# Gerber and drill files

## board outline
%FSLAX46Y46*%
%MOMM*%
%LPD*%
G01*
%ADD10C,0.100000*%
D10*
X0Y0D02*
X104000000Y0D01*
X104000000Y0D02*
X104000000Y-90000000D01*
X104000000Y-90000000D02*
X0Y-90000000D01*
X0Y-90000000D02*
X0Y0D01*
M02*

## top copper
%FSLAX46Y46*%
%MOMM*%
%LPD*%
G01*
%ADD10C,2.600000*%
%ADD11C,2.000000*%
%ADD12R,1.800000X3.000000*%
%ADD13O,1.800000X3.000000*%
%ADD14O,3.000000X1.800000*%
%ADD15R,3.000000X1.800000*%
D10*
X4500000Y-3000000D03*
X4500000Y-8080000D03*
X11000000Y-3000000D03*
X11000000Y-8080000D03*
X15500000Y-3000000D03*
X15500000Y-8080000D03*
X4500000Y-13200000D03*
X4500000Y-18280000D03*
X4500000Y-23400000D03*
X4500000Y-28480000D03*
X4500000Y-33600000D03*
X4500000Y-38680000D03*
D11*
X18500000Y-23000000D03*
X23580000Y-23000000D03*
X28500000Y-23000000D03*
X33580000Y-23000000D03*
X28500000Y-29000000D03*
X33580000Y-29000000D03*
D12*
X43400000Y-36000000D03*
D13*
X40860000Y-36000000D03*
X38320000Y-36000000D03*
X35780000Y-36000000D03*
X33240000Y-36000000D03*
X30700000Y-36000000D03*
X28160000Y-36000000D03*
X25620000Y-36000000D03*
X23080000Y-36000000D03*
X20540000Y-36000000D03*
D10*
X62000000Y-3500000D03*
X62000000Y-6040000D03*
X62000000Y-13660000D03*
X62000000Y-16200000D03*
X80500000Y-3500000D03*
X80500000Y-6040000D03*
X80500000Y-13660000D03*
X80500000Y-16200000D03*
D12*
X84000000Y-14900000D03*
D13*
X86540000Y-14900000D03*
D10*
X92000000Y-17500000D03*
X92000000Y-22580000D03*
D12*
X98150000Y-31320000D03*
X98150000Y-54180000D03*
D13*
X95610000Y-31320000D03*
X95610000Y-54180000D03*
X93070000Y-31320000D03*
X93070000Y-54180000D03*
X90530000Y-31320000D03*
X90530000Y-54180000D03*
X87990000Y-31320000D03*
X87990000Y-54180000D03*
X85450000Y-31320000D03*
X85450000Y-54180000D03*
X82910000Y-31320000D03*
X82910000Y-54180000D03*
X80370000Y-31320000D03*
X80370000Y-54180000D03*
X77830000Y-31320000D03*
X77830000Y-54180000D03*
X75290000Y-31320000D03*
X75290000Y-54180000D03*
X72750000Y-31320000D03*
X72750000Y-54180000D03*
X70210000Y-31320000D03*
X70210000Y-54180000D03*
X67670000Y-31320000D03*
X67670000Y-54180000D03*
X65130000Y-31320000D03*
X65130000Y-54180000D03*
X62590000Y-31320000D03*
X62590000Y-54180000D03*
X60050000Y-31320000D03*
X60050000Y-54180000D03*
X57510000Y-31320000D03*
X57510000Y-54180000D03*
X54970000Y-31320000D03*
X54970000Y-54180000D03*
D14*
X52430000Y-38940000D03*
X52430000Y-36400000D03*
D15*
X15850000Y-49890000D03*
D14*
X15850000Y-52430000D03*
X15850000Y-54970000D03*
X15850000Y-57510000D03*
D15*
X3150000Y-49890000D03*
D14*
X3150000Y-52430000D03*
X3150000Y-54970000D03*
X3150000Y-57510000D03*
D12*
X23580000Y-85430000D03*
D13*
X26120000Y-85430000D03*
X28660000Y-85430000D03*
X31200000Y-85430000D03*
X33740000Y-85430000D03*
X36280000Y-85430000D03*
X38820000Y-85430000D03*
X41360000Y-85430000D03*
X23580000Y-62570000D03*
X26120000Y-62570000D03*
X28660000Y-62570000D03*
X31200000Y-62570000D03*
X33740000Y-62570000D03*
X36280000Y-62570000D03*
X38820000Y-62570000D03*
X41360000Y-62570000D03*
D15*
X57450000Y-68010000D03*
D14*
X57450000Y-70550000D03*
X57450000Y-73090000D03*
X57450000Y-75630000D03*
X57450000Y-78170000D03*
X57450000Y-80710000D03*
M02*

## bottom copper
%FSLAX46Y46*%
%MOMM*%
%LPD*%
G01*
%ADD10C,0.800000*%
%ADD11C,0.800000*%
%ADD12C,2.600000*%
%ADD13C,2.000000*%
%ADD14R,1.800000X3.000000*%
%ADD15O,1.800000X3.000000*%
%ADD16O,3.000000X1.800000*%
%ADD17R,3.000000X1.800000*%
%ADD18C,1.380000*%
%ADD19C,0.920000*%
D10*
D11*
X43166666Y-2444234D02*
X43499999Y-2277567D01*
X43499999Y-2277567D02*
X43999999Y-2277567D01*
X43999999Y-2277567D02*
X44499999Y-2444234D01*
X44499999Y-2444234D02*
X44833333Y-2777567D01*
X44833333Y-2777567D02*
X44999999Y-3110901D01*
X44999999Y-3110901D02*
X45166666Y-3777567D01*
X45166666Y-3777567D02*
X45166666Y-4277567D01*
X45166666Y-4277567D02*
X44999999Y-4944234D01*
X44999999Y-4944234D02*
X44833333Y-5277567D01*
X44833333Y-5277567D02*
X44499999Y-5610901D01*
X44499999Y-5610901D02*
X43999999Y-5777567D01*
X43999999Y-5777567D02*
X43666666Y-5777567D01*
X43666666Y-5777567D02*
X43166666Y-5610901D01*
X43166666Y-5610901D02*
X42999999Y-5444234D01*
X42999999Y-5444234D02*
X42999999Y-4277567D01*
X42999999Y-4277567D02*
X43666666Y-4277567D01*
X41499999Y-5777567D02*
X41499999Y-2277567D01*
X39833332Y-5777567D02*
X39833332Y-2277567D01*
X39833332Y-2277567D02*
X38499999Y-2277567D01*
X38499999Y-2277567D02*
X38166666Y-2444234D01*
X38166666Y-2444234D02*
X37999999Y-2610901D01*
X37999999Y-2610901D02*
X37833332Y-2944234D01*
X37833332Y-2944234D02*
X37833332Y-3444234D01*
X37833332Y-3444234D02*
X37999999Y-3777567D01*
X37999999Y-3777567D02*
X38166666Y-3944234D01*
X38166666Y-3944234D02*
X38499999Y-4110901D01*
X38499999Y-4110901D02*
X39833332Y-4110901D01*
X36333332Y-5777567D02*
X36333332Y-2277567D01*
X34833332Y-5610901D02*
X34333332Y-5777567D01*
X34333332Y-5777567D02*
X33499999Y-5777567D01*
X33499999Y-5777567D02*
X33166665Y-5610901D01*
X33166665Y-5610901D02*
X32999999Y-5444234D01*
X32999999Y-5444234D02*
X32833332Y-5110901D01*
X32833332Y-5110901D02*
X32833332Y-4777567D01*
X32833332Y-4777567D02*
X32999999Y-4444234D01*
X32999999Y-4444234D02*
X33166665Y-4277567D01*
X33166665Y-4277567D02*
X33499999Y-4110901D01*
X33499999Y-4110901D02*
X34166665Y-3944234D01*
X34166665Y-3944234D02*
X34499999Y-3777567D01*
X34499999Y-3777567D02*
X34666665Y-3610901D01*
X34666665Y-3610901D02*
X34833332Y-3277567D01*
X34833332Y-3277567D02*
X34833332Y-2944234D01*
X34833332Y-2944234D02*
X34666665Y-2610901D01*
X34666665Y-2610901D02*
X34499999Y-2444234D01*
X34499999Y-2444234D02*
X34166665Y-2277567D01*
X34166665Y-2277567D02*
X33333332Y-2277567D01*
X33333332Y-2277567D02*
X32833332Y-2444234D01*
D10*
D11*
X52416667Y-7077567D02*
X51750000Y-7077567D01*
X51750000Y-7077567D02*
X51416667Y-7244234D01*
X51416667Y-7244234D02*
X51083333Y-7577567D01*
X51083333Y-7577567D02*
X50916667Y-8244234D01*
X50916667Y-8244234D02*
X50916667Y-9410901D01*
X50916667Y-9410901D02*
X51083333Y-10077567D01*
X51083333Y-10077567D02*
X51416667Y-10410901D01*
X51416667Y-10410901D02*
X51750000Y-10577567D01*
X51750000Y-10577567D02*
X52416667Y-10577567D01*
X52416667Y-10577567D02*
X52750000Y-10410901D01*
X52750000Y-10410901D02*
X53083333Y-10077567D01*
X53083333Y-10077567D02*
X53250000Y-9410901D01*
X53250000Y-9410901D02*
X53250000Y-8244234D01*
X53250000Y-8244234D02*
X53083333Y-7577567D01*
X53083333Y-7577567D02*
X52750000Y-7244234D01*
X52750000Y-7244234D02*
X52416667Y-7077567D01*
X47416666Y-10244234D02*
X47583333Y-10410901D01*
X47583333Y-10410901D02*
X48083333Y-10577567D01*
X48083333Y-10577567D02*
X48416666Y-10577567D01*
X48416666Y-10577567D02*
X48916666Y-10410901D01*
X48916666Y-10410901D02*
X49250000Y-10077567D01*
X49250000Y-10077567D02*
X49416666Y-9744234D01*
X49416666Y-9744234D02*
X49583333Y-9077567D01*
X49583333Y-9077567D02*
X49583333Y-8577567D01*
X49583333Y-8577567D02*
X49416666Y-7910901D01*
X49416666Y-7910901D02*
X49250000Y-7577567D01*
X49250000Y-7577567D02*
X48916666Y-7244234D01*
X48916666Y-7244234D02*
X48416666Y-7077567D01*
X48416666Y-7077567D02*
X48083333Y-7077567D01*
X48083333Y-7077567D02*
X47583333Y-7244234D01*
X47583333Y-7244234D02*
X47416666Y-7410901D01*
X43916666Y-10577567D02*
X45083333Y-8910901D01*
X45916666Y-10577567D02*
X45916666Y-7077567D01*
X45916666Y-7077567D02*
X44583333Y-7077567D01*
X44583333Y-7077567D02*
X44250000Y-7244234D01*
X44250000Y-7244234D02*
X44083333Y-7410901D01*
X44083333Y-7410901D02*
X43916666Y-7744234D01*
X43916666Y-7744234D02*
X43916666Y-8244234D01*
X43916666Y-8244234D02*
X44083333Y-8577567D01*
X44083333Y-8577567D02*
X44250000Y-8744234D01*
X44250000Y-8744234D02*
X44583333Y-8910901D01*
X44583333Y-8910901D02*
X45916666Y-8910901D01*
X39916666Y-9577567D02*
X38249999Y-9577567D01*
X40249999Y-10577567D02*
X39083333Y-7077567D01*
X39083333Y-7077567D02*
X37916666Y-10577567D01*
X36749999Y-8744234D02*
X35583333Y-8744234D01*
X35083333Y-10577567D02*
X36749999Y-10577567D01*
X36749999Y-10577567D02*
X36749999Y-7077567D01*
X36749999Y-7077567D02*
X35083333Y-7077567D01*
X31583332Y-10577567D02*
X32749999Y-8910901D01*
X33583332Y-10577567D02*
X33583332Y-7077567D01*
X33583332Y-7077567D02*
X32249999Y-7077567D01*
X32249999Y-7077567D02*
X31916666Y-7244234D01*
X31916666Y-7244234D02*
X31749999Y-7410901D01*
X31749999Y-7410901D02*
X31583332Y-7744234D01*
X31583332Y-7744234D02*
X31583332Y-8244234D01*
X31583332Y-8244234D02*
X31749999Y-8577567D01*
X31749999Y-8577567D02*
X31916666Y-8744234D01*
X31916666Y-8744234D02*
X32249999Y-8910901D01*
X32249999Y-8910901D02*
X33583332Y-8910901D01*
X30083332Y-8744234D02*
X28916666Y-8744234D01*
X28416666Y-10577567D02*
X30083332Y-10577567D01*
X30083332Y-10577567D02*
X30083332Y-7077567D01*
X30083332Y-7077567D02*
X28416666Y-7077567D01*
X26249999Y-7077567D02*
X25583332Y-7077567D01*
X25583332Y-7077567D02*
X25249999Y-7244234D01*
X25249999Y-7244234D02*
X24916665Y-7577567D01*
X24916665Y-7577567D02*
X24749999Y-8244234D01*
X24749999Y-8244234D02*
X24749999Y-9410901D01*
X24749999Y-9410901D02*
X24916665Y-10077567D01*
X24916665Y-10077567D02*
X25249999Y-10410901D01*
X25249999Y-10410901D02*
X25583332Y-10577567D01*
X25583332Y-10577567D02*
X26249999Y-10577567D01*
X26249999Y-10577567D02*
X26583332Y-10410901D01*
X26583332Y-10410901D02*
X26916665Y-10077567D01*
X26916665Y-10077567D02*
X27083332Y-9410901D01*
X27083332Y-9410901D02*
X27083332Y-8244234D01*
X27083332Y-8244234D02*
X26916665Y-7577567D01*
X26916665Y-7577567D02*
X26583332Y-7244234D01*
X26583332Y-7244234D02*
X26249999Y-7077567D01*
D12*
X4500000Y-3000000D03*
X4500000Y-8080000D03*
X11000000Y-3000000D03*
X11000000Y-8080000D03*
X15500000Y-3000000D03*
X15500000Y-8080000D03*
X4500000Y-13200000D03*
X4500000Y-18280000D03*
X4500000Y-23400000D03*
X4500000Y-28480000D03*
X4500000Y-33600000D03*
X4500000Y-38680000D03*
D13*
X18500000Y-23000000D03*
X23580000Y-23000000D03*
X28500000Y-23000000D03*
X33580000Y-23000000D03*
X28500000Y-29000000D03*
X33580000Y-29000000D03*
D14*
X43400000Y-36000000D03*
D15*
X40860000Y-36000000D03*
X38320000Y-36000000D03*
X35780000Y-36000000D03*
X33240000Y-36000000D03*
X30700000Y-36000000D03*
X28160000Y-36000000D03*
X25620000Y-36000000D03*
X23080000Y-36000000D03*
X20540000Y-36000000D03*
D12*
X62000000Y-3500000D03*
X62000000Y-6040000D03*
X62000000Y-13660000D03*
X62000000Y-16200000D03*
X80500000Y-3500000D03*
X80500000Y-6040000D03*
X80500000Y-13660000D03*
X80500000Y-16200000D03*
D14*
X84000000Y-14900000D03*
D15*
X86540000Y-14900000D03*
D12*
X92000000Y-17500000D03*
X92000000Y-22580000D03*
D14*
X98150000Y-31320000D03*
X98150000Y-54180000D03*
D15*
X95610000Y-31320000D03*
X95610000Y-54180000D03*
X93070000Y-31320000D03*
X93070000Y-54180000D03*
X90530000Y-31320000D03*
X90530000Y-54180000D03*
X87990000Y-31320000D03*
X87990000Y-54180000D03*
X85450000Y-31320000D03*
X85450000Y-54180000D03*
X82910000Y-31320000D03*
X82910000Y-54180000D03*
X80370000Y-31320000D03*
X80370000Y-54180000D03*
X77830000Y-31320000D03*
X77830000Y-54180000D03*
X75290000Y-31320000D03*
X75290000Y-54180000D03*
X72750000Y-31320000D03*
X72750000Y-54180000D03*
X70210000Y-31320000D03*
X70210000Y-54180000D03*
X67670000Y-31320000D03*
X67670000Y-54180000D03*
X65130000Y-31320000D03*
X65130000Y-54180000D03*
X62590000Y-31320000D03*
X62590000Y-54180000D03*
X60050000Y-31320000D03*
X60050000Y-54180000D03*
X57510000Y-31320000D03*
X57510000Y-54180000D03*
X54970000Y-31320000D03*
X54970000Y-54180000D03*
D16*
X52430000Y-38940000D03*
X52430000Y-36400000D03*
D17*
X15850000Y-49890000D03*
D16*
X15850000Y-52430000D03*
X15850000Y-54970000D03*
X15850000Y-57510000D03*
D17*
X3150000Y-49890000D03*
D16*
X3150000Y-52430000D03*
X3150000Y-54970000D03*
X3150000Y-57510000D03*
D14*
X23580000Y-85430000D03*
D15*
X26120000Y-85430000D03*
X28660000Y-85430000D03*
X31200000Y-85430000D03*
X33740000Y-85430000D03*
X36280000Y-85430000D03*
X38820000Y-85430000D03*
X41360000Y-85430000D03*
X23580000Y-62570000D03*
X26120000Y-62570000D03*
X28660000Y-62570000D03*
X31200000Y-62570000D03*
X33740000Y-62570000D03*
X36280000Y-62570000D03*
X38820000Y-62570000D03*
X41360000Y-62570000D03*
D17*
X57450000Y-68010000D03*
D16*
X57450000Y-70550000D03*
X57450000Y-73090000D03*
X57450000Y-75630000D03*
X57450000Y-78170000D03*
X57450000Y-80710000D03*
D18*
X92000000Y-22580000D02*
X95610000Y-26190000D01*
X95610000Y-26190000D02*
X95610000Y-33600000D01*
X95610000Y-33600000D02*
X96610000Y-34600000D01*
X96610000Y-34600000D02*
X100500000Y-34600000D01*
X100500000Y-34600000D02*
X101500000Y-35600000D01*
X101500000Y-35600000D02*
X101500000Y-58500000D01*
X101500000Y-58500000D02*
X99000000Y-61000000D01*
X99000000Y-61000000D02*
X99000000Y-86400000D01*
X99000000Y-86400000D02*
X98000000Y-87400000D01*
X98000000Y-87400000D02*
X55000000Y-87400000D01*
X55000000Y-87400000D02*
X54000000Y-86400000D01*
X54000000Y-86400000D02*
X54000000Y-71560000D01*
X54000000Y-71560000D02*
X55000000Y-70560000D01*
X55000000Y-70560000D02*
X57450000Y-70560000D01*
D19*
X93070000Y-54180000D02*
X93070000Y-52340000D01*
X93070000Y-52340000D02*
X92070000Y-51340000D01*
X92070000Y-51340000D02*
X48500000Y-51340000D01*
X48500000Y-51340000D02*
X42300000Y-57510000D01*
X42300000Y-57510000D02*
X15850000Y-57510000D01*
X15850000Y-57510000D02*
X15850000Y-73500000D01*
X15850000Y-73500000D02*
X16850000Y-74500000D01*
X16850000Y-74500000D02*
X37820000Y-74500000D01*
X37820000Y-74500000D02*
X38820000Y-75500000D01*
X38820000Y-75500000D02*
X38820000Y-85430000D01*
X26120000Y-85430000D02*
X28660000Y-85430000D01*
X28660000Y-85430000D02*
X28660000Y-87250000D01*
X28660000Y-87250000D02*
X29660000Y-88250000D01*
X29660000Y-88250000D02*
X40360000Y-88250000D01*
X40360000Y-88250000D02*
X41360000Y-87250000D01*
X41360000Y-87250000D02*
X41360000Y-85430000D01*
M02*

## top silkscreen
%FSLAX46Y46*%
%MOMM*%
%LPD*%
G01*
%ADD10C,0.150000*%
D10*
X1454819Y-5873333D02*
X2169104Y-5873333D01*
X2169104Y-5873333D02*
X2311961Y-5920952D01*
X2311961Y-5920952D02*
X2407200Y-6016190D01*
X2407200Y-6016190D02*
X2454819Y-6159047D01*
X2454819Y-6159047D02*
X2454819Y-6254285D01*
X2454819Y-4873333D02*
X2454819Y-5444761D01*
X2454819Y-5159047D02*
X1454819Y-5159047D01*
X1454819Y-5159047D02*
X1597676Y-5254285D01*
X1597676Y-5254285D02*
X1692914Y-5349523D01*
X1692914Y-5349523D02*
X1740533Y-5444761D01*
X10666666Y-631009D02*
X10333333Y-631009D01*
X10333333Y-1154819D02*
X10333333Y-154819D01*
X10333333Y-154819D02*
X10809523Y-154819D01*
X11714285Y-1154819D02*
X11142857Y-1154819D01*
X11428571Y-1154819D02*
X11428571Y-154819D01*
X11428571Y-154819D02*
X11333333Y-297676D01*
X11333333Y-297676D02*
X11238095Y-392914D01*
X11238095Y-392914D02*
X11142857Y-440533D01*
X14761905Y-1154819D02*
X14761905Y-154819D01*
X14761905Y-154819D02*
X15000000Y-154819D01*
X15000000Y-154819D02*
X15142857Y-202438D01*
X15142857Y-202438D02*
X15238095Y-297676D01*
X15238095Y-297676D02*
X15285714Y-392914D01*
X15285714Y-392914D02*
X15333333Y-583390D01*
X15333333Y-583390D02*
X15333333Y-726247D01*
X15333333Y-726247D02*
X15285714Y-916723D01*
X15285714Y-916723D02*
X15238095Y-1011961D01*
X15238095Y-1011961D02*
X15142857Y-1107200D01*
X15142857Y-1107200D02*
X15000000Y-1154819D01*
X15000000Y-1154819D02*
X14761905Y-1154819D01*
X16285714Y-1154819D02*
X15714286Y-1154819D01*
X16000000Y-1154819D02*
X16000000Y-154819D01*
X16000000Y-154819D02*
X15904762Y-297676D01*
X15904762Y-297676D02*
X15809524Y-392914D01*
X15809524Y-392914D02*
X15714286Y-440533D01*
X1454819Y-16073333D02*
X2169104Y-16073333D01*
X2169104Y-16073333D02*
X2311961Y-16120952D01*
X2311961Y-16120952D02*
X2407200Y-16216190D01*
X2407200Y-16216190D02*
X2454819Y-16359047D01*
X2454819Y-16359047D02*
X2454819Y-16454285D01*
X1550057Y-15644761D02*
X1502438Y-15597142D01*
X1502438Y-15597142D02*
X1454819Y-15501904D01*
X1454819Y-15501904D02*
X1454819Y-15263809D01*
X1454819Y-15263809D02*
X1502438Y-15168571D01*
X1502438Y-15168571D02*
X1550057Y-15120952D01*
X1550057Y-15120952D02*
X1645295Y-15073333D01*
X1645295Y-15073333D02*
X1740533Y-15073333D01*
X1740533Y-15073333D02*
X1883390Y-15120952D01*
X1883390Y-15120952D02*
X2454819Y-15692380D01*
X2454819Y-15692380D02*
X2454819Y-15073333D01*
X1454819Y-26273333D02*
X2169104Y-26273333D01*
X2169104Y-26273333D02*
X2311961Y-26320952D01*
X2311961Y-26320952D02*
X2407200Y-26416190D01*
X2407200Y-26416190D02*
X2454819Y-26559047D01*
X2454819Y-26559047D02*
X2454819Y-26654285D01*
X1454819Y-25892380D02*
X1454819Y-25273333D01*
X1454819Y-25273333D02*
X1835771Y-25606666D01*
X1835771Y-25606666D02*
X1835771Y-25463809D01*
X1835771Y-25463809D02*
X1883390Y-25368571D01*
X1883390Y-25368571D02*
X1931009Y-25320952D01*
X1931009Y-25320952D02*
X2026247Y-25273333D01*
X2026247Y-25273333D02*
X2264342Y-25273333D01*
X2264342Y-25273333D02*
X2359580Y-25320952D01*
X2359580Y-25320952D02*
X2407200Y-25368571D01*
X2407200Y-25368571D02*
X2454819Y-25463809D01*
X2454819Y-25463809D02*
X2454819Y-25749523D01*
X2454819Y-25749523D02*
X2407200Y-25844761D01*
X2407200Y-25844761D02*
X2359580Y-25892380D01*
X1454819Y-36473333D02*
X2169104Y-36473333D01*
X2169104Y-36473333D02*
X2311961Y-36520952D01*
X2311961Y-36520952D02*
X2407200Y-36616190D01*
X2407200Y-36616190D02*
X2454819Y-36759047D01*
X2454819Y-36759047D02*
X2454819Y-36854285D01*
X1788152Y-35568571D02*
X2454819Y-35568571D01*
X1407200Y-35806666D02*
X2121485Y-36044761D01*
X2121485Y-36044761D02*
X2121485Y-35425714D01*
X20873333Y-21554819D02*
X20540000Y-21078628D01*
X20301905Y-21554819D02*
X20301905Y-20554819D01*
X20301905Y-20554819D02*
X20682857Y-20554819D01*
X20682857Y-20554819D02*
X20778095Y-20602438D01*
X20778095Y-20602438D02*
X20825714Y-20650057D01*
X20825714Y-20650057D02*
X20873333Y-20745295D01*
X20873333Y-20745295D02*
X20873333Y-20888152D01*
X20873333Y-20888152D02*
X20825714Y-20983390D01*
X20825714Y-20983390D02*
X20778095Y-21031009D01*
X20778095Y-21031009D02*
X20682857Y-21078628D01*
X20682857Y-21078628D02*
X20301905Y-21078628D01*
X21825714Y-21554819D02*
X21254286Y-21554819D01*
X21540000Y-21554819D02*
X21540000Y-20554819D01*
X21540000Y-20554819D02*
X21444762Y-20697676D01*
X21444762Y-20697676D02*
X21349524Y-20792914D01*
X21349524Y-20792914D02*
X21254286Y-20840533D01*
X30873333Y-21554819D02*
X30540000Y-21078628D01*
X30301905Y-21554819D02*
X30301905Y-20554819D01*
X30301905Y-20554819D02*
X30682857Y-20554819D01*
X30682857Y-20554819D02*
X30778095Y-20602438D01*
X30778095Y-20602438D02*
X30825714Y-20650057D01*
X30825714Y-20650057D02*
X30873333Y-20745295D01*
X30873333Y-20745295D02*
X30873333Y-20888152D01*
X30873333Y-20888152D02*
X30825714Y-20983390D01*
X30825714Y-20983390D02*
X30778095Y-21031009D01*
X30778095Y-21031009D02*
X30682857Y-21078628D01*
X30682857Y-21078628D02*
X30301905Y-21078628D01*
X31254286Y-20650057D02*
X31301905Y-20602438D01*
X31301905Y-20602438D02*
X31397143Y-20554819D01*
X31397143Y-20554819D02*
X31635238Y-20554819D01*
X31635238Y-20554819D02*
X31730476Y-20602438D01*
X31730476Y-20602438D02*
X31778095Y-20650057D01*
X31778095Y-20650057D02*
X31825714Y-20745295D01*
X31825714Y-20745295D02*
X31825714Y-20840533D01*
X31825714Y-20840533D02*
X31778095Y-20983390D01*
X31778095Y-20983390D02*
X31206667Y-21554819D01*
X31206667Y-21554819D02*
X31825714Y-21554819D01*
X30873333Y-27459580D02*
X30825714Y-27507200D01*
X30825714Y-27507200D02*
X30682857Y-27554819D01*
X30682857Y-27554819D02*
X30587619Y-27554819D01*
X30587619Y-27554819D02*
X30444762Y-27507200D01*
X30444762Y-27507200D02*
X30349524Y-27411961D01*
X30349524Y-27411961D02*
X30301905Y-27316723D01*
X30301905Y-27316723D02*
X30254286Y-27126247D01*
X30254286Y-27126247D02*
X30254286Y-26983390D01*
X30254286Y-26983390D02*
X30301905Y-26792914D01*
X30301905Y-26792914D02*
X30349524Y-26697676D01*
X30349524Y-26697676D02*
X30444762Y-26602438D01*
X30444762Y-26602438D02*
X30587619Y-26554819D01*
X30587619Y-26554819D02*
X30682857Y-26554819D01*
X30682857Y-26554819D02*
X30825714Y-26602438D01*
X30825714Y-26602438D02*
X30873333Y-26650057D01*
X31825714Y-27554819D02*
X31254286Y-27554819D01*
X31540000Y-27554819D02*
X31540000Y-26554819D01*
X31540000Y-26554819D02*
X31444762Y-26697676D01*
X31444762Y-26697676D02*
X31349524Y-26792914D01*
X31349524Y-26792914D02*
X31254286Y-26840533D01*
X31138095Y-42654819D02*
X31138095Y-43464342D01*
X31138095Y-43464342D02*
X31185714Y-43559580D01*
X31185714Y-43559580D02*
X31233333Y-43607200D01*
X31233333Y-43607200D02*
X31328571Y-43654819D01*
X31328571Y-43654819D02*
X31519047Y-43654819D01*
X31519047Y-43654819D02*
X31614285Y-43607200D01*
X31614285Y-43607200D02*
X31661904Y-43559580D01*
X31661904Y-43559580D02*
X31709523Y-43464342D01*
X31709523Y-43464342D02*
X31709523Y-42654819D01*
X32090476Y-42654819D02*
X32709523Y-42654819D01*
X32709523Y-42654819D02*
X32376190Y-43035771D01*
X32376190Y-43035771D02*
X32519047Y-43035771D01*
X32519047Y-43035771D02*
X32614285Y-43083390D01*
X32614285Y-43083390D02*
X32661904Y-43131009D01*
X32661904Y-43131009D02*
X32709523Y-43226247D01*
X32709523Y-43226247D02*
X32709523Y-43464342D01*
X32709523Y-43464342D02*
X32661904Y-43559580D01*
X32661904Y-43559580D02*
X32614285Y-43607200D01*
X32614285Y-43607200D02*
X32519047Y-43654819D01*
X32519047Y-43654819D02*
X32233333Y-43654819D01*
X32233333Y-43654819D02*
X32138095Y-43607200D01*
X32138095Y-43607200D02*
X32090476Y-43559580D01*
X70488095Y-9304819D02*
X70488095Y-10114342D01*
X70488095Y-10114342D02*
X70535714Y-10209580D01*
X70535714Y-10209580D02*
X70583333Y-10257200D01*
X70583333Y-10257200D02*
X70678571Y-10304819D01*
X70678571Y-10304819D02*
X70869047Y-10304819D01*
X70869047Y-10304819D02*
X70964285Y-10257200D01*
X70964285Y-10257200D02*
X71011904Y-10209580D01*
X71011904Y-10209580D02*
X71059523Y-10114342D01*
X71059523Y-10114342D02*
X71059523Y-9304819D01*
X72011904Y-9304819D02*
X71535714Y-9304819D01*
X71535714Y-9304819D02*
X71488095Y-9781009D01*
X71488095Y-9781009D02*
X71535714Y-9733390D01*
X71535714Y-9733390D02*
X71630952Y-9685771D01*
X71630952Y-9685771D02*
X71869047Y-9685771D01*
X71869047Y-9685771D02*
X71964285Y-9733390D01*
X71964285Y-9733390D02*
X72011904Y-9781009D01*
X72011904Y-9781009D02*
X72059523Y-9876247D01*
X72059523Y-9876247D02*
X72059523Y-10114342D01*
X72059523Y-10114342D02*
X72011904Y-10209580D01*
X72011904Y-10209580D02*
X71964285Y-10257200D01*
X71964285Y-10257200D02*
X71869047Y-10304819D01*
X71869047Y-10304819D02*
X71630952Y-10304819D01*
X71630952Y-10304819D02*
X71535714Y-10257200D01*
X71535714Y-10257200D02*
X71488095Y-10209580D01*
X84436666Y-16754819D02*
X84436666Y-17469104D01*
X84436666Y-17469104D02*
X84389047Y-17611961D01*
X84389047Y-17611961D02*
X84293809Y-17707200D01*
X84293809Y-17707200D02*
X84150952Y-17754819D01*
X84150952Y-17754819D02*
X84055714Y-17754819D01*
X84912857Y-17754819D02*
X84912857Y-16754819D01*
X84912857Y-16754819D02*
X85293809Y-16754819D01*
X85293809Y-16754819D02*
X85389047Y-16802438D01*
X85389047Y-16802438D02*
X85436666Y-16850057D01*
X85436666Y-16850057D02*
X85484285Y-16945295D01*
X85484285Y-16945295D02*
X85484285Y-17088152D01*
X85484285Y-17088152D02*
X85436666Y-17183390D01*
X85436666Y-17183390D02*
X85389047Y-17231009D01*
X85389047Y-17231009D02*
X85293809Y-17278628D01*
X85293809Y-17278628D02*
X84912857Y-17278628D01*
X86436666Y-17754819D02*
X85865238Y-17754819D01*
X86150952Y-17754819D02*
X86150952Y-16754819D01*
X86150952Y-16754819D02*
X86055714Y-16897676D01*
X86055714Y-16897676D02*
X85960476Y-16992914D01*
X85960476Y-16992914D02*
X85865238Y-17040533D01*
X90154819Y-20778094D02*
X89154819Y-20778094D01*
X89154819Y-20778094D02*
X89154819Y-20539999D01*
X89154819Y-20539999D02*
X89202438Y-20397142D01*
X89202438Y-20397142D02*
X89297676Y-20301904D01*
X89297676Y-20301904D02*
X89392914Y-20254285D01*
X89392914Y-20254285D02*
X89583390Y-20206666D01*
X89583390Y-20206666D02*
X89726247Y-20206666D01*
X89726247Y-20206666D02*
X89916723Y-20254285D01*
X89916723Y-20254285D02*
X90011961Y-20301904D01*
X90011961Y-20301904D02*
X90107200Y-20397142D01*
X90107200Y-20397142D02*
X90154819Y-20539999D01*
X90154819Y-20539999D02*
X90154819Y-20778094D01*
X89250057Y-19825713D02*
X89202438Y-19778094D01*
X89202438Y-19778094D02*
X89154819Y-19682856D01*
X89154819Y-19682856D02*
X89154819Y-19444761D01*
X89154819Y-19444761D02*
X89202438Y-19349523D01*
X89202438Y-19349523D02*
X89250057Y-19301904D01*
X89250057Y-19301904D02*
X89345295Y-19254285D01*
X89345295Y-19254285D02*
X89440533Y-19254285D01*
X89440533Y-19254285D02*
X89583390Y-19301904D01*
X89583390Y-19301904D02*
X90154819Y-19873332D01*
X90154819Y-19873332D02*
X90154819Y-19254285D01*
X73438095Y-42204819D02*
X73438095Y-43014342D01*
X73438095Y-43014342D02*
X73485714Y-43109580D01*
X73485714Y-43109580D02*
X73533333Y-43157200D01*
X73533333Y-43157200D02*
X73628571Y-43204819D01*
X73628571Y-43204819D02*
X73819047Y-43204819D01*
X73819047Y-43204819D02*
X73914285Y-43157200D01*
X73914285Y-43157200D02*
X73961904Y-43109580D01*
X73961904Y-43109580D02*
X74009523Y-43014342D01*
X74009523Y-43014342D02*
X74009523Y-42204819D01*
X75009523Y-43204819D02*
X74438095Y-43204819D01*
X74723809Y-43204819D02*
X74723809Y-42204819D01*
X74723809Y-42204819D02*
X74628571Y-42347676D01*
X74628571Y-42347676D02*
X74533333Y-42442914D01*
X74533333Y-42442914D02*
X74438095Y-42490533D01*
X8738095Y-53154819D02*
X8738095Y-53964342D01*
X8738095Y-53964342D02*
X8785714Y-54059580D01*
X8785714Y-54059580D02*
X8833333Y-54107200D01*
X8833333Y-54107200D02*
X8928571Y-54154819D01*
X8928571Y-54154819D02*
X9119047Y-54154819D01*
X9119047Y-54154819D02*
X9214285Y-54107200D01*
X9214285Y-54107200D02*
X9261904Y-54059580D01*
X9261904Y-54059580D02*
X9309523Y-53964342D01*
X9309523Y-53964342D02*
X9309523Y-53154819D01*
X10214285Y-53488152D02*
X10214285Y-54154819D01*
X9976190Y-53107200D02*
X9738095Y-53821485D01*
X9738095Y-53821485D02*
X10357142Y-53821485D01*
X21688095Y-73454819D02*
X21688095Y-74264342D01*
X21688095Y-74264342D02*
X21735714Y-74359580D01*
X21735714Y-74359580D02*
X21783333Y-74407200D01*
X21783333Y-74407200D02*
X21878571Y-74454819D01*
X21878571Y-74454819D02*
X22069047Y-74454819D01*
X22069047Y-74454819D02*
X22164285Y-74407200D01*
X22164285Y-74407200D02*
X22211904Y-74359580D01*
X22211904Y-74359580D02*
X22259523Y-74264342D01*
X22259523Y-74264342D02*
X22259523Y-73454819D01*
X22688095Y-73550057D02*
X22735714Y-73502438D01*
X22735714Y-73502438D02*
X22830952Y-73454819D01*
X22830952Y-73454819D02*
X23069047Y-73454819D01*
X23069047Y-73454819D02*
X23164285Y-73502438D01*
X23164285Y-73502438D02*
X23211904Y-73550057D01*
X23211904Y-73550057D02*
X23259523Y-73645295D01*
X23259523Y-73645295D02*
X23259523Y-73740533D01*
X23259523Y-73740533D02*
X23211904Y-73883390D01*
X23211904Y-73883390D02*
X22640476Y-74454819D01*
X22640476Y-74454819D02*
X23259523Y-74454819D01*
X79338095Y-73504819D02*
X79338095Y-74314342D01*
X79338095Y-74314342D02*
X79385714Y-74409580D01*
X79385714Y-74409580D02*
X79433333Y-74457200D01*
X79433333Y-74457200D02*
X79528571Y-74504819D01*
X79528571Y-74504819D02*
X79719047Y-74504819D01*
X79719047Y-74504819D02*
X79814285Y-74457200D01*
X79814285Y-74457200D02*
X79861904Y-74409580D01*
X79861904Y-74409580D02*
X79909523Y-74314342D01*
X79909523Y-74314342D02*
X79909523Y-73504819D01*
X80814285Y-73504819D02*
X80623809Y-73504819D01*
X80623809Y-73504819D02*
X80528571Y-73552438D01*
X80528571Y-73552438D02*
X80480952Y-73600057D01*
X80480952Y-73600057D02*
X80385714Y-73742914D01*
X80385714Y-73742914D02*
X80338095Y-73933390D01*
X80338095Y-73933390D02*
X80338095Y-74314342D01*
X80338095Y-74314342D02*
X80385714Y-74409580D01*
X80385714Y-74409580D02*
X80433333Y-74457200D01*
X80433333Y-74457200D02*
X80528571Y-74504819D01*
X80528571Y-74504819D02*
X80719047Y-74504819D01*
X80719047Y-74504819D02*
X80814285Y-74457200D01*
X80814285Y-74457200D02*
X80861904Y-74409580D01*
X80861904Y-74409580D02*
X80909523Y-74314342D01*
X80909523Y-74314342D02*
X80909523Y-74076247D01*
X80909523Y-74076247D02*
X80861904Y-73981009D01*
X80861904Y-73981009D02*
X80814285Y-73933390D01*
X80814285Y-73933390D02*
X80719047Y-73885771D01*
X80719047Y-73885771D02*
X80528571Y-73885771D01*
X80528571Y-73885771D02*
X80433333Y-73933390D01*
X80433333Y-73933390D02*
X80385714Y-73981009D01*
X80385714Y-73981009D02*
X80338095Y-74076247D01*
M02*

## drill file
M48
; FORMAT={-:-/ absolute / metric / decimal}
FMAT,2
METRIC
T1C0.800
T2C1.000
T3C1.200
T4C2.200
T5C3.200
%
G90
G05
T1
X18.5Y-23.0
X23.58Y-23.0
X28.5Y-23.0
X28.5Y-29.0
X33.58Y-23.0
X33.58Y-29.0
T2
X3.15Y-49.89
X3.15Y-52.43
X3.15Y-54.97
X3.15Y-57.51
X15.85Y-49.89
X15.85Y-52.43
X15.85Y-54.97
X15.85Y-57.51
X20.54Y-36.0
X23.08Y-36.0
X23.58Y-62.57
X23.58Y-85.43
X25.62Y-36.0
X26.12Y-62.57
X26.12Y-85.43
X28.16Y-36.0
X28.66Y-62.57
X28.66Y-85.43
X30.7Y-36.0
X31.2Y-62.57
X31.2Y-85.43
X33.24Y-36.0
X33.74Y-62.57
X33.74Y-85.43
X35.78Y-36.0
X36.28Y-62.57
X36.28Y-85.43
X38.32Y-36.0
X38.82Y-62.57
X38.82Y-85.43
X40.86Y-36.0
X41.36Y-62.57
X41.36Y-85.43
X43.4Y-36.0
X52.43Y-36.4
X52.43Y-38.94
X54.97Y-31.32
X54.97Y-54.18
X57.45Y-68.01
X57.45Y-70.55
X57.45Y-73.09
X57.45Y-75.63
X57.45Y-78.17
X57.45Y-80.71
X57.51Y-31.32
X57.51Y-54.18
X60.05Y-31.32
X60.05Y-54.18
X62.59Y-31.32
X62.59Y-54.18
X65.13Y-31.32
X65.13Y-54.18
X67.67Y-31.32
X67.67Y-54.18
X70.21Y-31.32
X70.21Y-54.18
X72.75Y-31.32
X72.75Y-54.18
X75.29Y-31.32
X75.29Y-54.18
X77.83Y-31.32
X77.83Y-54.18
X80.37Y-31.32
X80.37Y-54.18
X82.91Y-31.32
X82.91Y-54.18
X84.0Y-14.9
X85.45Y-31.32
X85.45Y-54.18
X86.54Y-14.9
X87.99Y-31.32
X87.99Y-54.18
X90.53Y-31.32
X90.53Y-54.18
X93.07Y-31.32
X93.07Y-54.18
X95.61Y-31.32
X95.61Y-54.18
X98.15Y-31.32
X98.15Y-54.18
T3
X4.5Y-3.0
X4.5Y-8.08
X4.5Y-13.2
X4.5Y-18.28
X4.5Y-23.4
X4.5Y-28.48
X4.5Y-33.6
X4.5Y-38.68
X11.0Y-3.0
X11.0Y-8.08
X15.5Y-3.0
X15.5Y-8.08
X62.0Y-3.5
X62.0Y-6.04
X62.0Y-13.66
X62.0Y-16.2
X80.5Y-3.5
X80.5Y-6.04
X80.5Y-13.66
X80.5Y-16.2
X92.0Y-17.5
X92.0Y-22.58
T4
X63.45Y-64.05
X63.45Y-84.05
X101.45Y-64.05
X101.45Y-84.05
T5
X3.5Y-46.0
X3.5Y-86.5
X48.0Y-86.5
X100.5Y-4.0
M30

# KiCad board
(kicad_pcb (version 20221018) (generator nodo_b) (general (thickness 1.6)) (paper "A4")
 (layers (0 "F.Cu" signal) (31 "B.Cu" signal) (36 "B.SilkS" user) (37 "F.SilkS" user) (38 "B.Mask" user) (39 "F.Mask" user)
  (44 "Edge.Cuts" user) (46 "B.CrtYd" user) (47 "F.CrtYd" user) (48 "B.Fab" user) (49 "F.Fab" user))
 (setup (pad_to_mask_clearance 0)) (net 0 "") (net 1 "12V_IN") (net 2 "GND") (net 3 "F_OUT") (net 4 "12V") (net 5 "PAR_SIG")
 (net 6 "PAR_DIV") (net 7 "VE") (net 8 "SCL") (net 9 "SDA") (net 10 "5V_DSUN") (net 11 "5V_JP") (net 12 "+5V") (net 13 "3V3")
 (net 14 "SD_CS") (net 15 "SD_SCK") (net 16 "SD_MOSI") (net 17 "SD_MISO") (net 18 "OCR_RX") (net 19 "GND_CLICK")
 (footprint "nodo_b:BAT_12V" (layer "F.Cu") (at 4.5 3.0)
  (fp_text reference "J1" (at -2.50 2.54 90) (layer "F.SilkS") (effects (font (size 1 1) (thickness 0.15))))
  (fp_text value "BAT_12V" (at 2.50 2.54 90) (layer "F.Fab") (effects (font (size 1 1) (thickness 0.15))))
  (pad "1" thru_hole circle (at 0 0.0) (size 2.6 2.6) (drill 1.2) (layers "*.Cu" "*.Mask") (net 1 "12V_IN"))
  (pad "2" thru_hole circle (at 0 5.08) (size 2.6 2.6) (drill 1.2) (layers "*.Cu" "*.Mask") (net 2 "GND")))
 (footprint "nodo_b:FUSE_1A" (layer "F.Cu") (at 11.0 3.0)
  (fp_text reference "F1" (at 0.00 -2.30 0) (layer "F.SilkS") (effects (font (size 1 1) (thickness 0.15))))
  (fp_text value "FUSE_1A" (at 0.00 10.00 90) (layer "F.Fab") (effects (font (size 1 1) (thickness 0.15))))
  (pad "1" thru_hole circle (at 0 0) (size 2.6 2.6) (drill 1.2) (layers "*.Cu" "*.Mask") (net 1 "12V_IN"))
  (pad "2" thru_hole circle (at 0 5.08) (size 2.6 2.6) (drill 1.2) (layers "*.Cu" "*.Mask") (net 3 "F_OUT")))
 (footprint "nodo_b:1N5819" (layer "F.Cu") (at 15.5 3.0)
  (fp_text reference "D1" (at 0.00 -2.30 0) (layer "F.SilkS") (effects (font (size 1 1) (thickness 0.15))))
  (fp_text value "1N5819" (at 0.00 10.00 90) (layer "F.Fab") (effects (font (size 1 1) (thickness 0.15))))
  (pad "1" thru_hole circle (at 0 0) (size 2.6 2.6) (drill 1.2) (layers "*.Cu" "*.Mask") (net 3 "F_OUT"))
  (pad "2" thru_hole circle (at 0 5.08) (size 2.6 2.6) (drill 1.2) (layers "*.Cu" "*.Mask") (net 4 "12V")))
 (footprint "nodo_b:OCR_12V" (layer "F.Cu") (at 4.5 13.2)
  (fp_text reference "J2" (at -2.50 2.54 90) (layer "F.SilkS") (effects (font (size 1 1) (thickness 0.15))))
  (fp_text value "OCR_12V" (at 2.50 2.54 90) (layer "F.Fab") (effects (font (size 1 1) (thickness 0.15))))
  (pad "1" thru_hole circle (at 0 0.0) (size 2.6 2.6) (drill 1.2) (layers "*.Cu" "*.Mask") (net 2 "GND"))
  (pad "2" thru_hole circle (at 0 5.08) (size 2.6 2.6) (drill 1.2) (layers "*.Cu" "*.Mask") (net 4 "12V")))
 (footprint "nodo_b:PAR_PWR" (layer "F.Cu") (at 4.5 23.4)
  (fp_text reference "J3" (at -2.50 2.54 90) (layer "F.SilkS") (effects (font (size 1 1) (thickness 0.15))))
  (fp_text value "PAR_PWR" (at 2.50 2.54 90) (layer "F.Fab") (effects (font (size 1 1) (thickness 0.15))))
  (pad "1" thru_hole circle (at 0 0.0) (size 2.6 2.6) (drill 1.2) (layers "*.Cu" "*.Mask") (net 4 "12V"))
  (pad "2" thru_hole circle (at 0 5.08) (size 2.6 2.6) (drill 1.2) (layers "*.Cu" "*.Mask") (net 2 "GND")))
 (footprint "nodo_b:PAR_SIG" (layer "F.Cu") (at 4.5 33.6)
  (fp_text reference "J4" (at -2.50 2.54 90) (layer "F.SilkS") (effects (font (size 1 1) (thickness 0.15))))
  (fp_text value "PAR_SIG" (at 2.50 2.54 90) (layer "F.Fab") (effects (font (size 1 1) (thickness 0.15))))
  (pad "1" thru_hole circle (at 0 0.0) (size 2.6 2.6) (drill 1.2) (layers "*.Cu" "*.Mask") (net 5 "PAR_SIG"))
  (pad "2" thru_hole circle (at 0 5.08) (size 2.6 2.6) (drill 1.2) (layers "*.Cu" "*.Mask") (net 2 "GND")))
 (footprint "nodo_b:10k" (layer "F.Cu") (at 18.5 23.0)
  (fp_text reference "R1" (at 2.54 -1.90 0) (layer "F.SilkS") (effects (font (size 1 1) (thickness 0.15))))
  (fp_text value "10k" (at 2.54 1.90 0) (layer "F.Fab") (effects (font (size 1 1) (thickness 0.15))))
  (pad "1" thru_hole circle (at 0 0) (size 2.0 2.0) (drill 0.8) (layers "*.Cu" "*.Mask") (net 5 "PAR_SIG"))
  (pad "2" thru_hole circle (at 5.08 0) (size 2.0 2.0) (drill 0.8) (layers "*.Cu" "*.Mask") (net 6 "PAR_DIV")))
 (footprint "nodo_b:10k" (layer "F.Cu") (at 28.5 23.0)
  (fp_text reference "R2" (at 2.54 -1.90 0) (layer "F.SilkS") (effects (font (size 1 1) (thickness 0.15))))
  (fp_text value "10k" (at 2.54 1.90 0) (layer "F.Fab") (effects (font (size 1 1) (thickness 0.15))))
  (pad "1" thru_hole circle (at 0 0) (size 2.0 2.0) (drill 0.8) (layers "*.Cu" "*.Mask") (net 2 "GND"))
  (pad "2" thru_hole circle (at 5.08 0) (size 2.0 2.0) (drill 0.8) (layers "*.Cu" "*.Mask") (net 6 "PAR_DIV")))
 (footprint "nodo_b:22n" (layer "F.Cu") (at 28.5 29.0)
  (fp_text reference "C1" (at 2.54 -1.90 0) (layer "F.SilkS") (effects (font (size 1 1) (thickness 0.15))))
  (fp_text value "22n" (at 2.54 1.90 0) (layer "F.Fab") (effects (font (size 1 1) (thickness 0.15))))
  (pad "1" thru_hole circle (at 0 0) (size 2.0 2.0) (drill 0.8) (layers "*.Cu" "*.Mask") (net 6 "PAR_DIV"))
  (pad "2" thru_hole circle (at 5.08 0) (size 2.0 2.0) (drill 0.8) (layers "*.Cu" "*.Mask") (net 2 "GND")))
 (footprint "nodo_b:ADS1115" (layer "F.Cu") (at 43.4 36.0 180)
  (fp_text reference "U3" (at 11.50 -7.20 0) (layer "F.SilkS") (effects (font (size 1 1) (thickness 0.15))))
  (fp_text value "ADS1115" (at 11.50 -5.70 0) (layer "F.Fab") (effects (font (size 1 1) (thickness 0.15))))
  (pad "1" thru_hole rect (at 0.0 0 180) (size 1.8 3.0) (drill 1.0) (layers "*.Cu" "*.Mask") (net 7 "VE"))
  (pad "2" thru_hole oval (at 2.54 0 180) (size 1.8 3.0) (drill 1.0) (layers "*.Cu" "*.Mask") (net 2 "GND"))
  (pad "3" thru_hole oval (at 5.08 0 180) (size 1.8 3.0) (drill 1.0) (layers "*.Cu" "*.Mask") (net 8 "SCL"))
  (pad "4" thru_hole oval (at 7.62 0 180) (size 1.8 3.0) (drill 1.0) (layers "*.Cu" "*.Mask") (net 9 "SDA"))
  (pad "5" thru_hole oval (at 10.16 0 180) (size 1.8 3.0) (drill 1.0) (layers "*.Cu" "*.Mask") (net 2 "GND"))
  (pad "6" thru_hole oval (at 12.7 0 180) (size 1.8 3.0) (drill 1.0) (layers "*.Cu" "*.Mask"))
  (pad "7" thru_hole oval (at 15.24 0 180) (size 1.8 3.0) (drill 1.0) (layers "*.Cu" "*.Mask") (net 6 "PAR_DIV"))
  (pad "8" thru_hole oval (at 17.78 0 180) (size 1.8 3.0) (drill 1.0) (layers "*.Cu" "*.Mask"))
  (pad "9" thru_hole oval (at 20.32 0 180) (size 1.8 3.0) (drill 1.0) (layers "*.Cu" "*.Mask"))
  (pad "10" thru_hole oval (at 22.86 0 180) (size 1.8 3.0) (drill 1.0) (layers "*.Cu" "*.Mask")))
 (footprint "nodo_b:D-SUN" (layer "F.Cu") (at 62.0 3.5)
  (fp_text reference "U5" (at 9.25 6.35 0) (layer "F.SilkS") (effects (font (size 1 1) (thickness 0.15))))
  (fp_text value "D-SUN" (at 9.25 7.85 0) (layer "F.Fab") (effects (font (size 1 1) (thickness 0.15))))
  (pad "1" thru_hole circle (at 0 0.0) (size 2.6 2.6) (drill 1.2) (layers "*.Cu" "*.Mask") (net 2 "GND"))
  (pad "2" thru_hole circle (at 0 2.54) (size 2.6 2.6) (drill 1.2) (layers "*.Cu" "*.Mask") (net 2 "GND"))
  (pad "3" thru_hole circle (at 0 10.16) (size 2.6 2.6) (drill 1.2) (layers "*.Cu" "*.Mask") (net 4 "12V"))
  (pad "4" thru_hole circle (at 0 12.7) (size 2.6 2.6) (drill 1.2) (layers "*.Cu" "*.Mask") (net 4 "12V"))
  (pad "5" thru_hole circle (at 18.5 0.0) (size 2.6 2.6) (drill 1.2) (layers "*.Cu" "*.Mask") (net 2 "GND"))
  (pad "6" thru_hole circle (at 18.5 2.54) (size 2.6 2.6) (drill 1.2) (layers "*.Cu" "*.Mask") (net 2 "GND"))
  (pad "7" thru_hole circle (at 18.5 10.16) (size 2.6 2.6) (drill 1.2) (layers "*.Cu" "*.Mask") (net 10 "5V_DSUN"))
  (pad "8" thru_hole circle (at 18.5 12.7) (size 2.6 2.6) (drill 1.2) (layers "*.Cu" "*.Mask") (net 10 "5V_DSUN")))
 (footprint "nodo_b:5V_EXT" (layer "F.Cu") (at 84.0 14.9)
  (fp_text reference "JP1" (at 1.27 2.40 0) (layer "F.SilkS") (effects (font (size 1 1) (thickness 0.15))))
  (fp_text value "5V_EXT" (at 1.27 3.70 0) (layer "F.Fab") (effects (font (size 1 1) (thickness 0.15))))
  (pad "1" thru_hole rect (at 0.0 0) (size 1.8 3.0) (drill 1.0) (layers "*.Cu" "*.Mask") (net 10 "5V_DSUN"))
  (pad "2" thru_hole oval (at 2.54 0) (size 1.8 3.0) (drill 1.0) (layers "*.Cu" "*.Mask") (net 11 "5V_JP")))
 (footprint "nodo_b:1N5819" (layer "F.Cu") (at 92.0 17.5)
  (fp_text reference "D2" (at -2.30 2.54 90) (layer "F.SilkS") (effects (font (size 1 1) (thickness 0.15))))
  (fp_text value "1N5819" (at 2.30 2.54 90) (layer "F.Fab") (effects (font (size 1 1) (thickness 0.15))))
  (pad "1" thru_hole circle (at 0 0) (size 2.6 2.6) (drill 1.2) (layers "*.Cu" "*.Mask") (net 11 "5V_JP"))
  (pad "2" thru_hole circle (at 0 5.08) (size 2.6 2.6) (drill 1.2) (layers "*.Cu" "*.Mask") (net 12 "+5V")))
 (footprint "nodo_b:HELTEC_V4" (layer "F.Cu") (at 47.900000000000006 30.0)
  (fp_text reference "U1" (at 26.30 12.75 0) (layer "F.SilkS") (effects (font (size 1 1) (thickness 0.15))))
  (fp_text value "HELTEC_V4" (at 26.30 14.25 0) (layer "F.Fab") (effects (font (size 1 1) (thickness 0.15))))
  (pad "A1" thru_hole rect (at 50.25 1.32) (size 1.8 3.0) (drill 1.0) (layers "*.Cu" "*.Mask") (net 2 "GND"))
  (pad "B1" thru_hole rect (at 50.25 24.18) (size 1.8 3.0) (drill 1.0) (layers "*.Cu" "*.Mask"))
  (pad "A2" thru_hole oval (at 47.71 1.32) (size 1.8 3.0) (drill 1.0) (layers "*.Cu" "*.Mask") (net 12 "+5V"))
  (pad "B2" thru_hole oval (at 47.71 24.18) (size 1.8 3.0) (drill 1.0) (layers "*.Cu" "*.Mask") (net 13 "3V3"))
  (pad "A3" thru_hole oval (at 45.17 1.32) (size 1.8 3.0) (drill 1.0) (layers "*.Cu" "*.Mask") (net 7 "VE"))
  (pad "B3" thru_hole oval (at 45.17 24.18) (size 1.8 3.0) (drill 1.0) (layers "*.Cu" "*.Mask") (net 13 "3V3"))
  (pad "A4" thru_hole oval (at 42.63 1.32) (size 1.8 3.0) (drill 1.0) (layers "*.Cu" "*.Mask") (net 7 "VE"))
  (pad "B4" thru_hole oval (at 42.63 24.18) (size 1.8 3.0) (drill 1.0) (layers "*.Cu" "*.Mask"))
  (pad "A5" thru_hole oval (at 40.09 1.32) (size 1.8 3.0) (drill 1.0) (layers "*.Cu" "*.Mask"))
  (pad "B5" thru_hole oval (at 40.09 24.18) (size 1.8 3.0) (drill 1.0) (layers "*.Cu" "*.Mask"))
  (pad "A6" thru_hole oval (at 37.55 1.32) (size 1.8 3.0) (drill 1.0) (layers "*.Cu" "*.Mask"))
  (pad "B6" thru_hole oval (at 37.55 24.18) (size 1.8 3.0) (drill 1.0) (layers "*.Cu" "*.Mask"))
  (pad "A7" thru_hole oval (at 35.01 1.32) (size 1.8 3.0) (drill 1.0) (layers "*.Cu" "*.Mask"))
  (pad "B7" thru_hole oval (at 35.01 24.18) (size 1.8 3.0) (drill 1.0) (layers "*.Cu" "*.Mask") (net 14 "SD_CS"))
  (pad "A8" thru_hole oval (at 32.47 1.32) (size 1.8 3.0) (drill 1.0) (layers "*.Cu" "*.Mask"))
  (pad "B8" thru_hole oval (at 32.47 24.18) (size 1.8 3.0) (drill 1.0) (layers "*.Cu" "*.Mask") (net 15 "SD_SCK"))
  (pad "A9" thru_hole oval (at 29.93 1.32) (size 1.8 3.0) (drill 1.0) (layers "*.Cu" "*.Mask"))
  (pad "B9" thru_hole oval (at 29.93 24.18) (size 1.8 3.0) (drill 1.0) (layers "*.Cu" "*.Mask") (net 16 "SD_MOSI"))
  (pad "A10" thru_hole oval (at 27.39 1.32) (size 1.8 3.0) (drill 1.0) (layers "*.Cu" "*.Mask"))
  (pad "B10" thru_hole oval (at 27.39 24.18) (size 1.8 3.0) (drill 1.0) (layers "*.Cu" "*.Mask") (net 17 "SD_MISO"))
  (pad "A11" thru_hole oval (at 24.85 1.32) (size 1.8 3.0) (drill 1.0) (layers "*.Cu" "*.Mask"))
  (pad "B11" thru_hole oval (at 24.85 24.18) (size 1.8 3.0) (drill 1.0) (layers "*.Cu" "*.Mask"))
  (pad "A12" thru_hole oval (at 22.31 1.32) (size 1.8 3.0) (drill 1.0) (layers "*.Cu" "*.Mask"))
  (pad "B12" thru_hole oval (at 22.31 24.18) (size 1.8 3.0) (drill 1.0) (layers "*.Cu" "*.Mask"))
  (pad "A13" thru_hole oval (at 19.77 1.32) (size 1.8 3.0) (drill 1.0) (layers "*.Cu" "*.Mask"))
  (pad "B13" thru_hole oval (at 19.77 24.18) (size 1.8 3.0) (drill 1.0) (layers "*.Cu" "*.Mask"))
  (pad "A14" thru_hole oval (at 17.229999999999997 1.32) (size 1.8 3.0) (drill 1.0) (layers "*.Cu" "*.Mask"))
  (pad "B14" thru_hole oval (at 17.229999999999997 24.18) (size 1.8 3.0) (drill 1.0) (layers "*.Cu" "*.Mask"))
  (pad "A15" thru_hole oval (at 14.689999999999998 1.32) (size 1.8 3.0) (drill 1.0) (layers "*.Cu" "*.Mask"))
  (pad "B15" thru_hole oval (at 14.689999999999998 24.18) (size 1.8 3.0) (drill 1.0) (layers "*.Cu" "*.Mask"))
  (pad "A16" thru_hole oval (at 12.149999999999999 1.32) (size 1.8 3.0) (drill 1.0) (layers "*.Cu" "*.Mask"))
  (pad "B16" thru_hole oval (at 12.149999999999999 24.18) (size 1.8 3.0) (drill 1.0) (layers "*.Cu" "*.Mask"))
  (pad "A17" thru_hole oval (at 9.61 1.32) (size 1.8 3.0) (drill 1.0) (layers "*.Cu" "*.Mask"))
  (pad "B17" thru_hole oval (at 9.61 24.18) (size 1.8 3.0) (drill 1.0) (layers "*.Cu" "*.Mask") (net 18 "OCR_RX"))
  (pad "A18" thru_hole oval (at 7.07 1.32) (size 1.8 3.0) (drill 1.0) (layers "*.Cu" "*.Mask"))
  (pad "B18" thru_hole oval (at 7.07 24.18) (size 1.8 3.0) (drill 1.0) (layers "*.Cu" "*.Mask"))
  (pad "AUX17" thru_hole oval (at 4.530000000000001 8.94) (size 3.0 1.8) (drill 1.0) (layers "*.Cu" "*.Mask") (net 9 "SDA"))
  (pad "AUX18" thru_hole oval (at 4.530000000000001 6.4) (size 3.0 1.8) (drill 1.0) (layers "*.Cu" "*.Mask") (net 8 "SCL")))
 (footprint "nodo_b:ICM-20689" (layer "F.Cu") (at 2.0 48.0)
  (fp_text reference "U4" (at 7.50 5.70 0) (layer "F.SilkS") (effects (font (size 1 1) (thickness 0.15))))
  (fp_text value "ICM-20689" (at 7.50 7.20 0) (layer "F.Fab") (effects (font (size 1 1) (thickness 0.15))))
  (pad "1" thru_hole rect (at 13.85 1.89) (size 3.0 1.8) (drill 1.0) (layers "*.Cu" "*.Mask") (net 9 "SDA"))
  (pad "2" thru_hole oval (at 13.85 4.43) (size 3.0 1.8) (drill 1.0) (layers "*.Cu" "*.Mask") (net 8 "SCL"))
  (pad "3" thru_hole oval (at 13.85 6.97) (size 3.0 1.8) (drill 1.0) (layers "*.Cu" "*.Mask") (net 2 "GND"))
  (pad "4" thru_hole oval (at 13.85 9.51) (size 3.0 1.8) (drill 1.0) (layers "*.Cu" "*.Mask") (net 13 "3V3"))
  (pad "5" thru_hole rect (at 1.15 1.89) (size 3.0 1.8) (drill 1.0) (layers "*.Cu" "*.Mask") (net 2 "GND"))
  (pad "6" thru_hole oval (at 1.15 4.43) (size 3.0 1.8) (drill 1.0) (layers "*.Cu" "*.Mask"))
  (pad "7" thru_hole oval (at 1.15 6.97) (size 3.0 1.8) (drill 1.0) (layers "*.Cu" "*.Mask"))
  (pad "8" thru_hole oval (at 1.15 9.51) (size 3.0 1.8) (drill 1.0) (layers "*.Cu" "*.Mask")))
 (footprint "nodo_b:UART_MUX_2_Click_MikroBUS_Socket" (layer "F.Cu") (at 43.9 74.0 90)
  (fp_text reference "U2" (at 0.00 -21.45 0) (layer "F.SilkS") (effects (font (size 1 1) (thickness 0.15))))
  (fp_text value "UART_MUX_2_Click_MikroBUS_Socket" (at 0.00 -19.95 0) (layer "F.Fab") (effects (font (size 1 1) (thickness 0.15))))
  (pad "1" thru_hole rect (at -11.43 -20.32 90) (size 3.0 1.8) (drill 1.0) (layers "*.Cu" "*.Mask"))
  (pad "2" thru_hole oval (at -11.43 -17.78 90) (size 3.0 1.8) (drill 1.0) (layers "*.Cu" "*.Mask") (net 2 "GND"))
  (pad "3" thru_hole oval (at -11.43 -15.24 90) (size 3.0 1.8) (drill 1.0) (layers "*.Cu" "*.Mask") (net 2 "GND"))
  (pad "4" thru_hole oval (at -11.43 -12.7 90) (size 3.0 1.8) (drill 1.0) (layers "*.Cu" "*.Mask"))
  (pad "5" thru_hole oval (at -11.43 -10.16 90) (size 3.0 1.8) (drill 1.0) (layers "*.Cu" "*.Mask"))
  (pad "6" thru_hole oval (at -11.43 -7.620000000000001 90) (size 3.0 1.8) (drill 1.0) (layers "*.Cu" "*.Mask"))
  (pad "7" thru_hole oval (at -11.43 -5.08 90) (size 3.0 1.8) (drill 1.0) (layers "*.Cu" "*.Mask") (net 13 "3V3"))
  (pad "8" thru_hole oval (at -11.43 -2.539999999999999 90) (size 3.0 1.8) (drill 1.0) (layers "*.Cu" "*.Mask") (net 2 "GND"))
  (pad "16" thru_hole oval (at 11.43 -20.32 90) (size 3.0 1.8) (drill 1.0) (layers "*.Cu" "*.Mask"))
  (pad "15" thru_hole oval (at 11.43 -17.78 90) (size 3.0 1.8) (drill 1.0) (layers "*.Cu" "*.Mask"))
  (pad "14" thru_hole oval (at 11.43 -15.239999999999998 90) (size 3.0 1.8) (drill 1.0) (layers "*.Cu" "*.Mask") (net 18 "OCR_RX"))
  (pad "13" thru_hole oval (at 11.43 -12.7 90) (size 3.0 1.8) (drill 1.0) (layers "*.Cu" "*.Mask"))
  (pad "12" thru_hole oval (at 11.43 -10.16 90) (size 3.0 1.8) (drill 1.0) (layers "*.Cu" "*.Mask"))
  (pad "11" thru_hole oval (at 11.43 -7.62 90) (size 3.0 1.8) (drill 1.0) (layers "*.Cu" "*.Mask"))
  (pad "10" thru_hole oval (at 11.43 -5.08 90) (size 3.0 1.8) (drill 1.0) (layers "*.Cu" "*.Mask"))
  (pad "9" thru_hole oval (at 11.43 -2.54 90) (size 3.0 1.8) (drill 1.0) (layers "*.Cu" "*.Mask")))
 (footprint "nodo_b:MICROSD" (layer "F.Cu") (at 61.4 62.0)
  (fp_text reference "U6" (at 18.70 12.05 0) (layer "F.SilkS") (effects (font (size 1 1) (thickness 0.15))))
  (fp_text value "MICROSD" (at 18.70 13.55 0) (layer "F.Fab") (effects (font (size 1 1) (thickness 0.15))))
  (pad "1" thru_hole rect (at -3.95 6.01) (size 3.0 1.8) (drill 1.0) (layers "*.Cu" "*.Mask") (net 2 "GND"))
  (pad "2" thru_hole oval (at -3.95 8.55) (size 3.0 1.8) (drill 1.0) (layers "*.Cu" "*.Mask") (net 12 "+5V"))
  (pad "3" thru_hole oval (at -3.95 11.09) (size 3.0 1.8) (drill 1.0) (layers "*.Cu" "*.Mask") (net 17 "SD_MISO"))
  (pad "4" thru_hole oval (at -3.95 13.629999999999999) (size 3.0 1.8) (drill 1.0) (layers "*.Cu" "*.Mask") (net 16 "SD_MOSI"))
  (pad "5" thru_hole oval (at -3.95 16.17) (size 3.0 1.8) (drill 1.0) (layers "*.Cu" "*.Mask") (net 15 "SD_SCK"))
  (pad "6" thru_hole oval (at -3.95 18.71) (size 3.0 1.8) (drill 1.0) (layers "*.Cu" "*.Mask") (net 14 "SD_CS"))
  (pad "" np_thru_hole circle (at 2.05 2.05) (size 2.2 2.2) (drill 2.2) (layers "*.Cu" "*.Mask"))
  (pad "" np_thru_hole circle (at 40.05 2.05) (size 2.2 2.2) (drill 2.2) (layers "*.Cu" "*.Mask"))
  (pad "" np_thru_hole circle (at 2.05 22.05) (size 2.2 2.2) (drill 2.2) (layers "*.Cu" "*.Mask"))
  (pad "" np_thru_hole circle (at 40.05 22.05) (size 2.2 2.2) (drill 2.2) (layers "*.Cu" "*.Mask")))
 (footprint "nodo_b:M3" (layer "F.Cu") (at 3.5 86.5)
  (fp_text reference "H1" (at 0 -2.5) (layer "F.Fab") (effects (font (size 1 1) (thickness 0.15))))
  (pad "" np_thru_hole circle (at 0 0) (size 3.2 3.2) (drill 3.2) (layers "*.Cu" "*.Mask")))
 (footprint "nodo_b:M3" (layer "F.Cu") (at 48.0 86.5)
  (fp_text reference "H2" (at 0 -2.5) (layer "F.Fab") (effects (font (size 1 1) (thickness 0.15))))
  (pad "" np_thru_hole circle (at 0 0) (size 3.2 3.2) (drill 3.2) (layers "*.Cu" "*.Mask")))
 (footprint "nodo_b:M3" (layer "F.Cu") (at 3.5 46.0)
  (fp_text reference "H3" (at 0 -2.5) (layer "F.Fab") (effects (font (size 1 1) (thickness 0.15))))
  (pad "" np_thru_hole circle (at 0 0) (size 3.2 3.2) (drill 3.2) (layers "*.Cu" "*.Mask")))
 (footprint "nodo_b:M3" (layer "F.Cu") (at 100.5 4.0)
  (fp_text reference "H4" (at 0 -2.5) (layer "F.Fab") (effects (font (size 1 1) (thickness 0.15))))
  (pad "" np_thru_hole circle (at 0 0) (size 3.2 3.2) (drill 3.2) (layers "*.Cu" "*.Mask")))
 (segment locked (start 92.0 22.58) (end 95.61 26.19) (width 1.38) (layer "B.Cu") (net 12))
 (segment locked (start 95.61 26.19) (end 95.61 33.6) (width 1.38) (layer "B.Cu") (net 12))
 (segment locked (start 95.61 33.6) (end 96.61 34.6) (width 1.38) (layer "B.Cu") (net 12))
 (segment locked (start 96.61 34.6) (end 100.5 34.6) (width 1.38) (layer "B.Cu") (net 12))
 (segment locked (start 100.5 34.6) (end 101.5 35.6) (width 1.38) (layer "B.Cu") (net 12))
 (segment locked (start 101.5 35.6) (end 101.5 58.5) (width 1.38) (layer "B.Cu") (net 12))
 (segment locked (start 101.5 58.5) (end 99.0 61.0) (width 1.38) (layer "B.Cu") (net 12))
 (segment locked (start 99.0 61.0) (end 99.0 86.4) (width 1.38) (layer "B.Cu") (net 12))
 (segment locked (start 99.0 86.4) (end 98.0 87.4) (width 1.38) (layer "B.Cu") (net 12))
 (segment locked (start 98.0 87.4) (end 55.0 87.4) (width 1.38) (layer "B.Cu") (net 12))
 (segment locked (start 55.0 87.4) (end 54.0 86.4) (width 1.38) (layer "B.Cu") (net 12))
 (segment locked (start 54.0 86.4) (end 54.0 71.56) (width 1.38) (layer "B.Cu") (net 12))
 (segment locked (start 54.0 71.56) (end 55.0 70.56) (width 1.38) (layer "B.Cu") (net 12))
 (segment locked (start 55.0 70.56) (end 57.449999999999996 70.56) (width 1.38) (layer "B.Cu") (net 12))
 (segment locked (start 93.07 54.18) (end 93.07 52.34) (width 0.92) (layer "B.Cu") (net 13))
 (segment locked (start 93.07 52.34) (end 92.07 51.34) (width 0.92) (layer "B.Cu") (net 13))
 (segment locked (start 92.07 51.34) (end 48.5 51.34) (width 0.92) (layer "B.Cu") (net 13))
 (segment locked (start 48.5 51.34) (end 42.3 57.51) (width 0.92) (layer "B.Cu") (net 13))
 (segment locked (start 42.3 57.51) (end 15.85 57.51) (width 0.92) (layer "B.Cu") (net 13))
 (segment locked (start 15.85 57.51) (end 15.85 73.5) (width 0.92) (layer "B.Cu") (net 13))
 (segment locked (start 15.85 73.5) (end 16.85 74.5) (width 0.92) (layer "B.Cu") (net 13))
 (segment locked (start 16.85 74.5) (end 37.82 74.5) (width 0.92) (layer "B.Cu") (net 13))
 (segment locked (start 37.82 74.5) (end 38.82 75.5) (width 0.92) (layer "B.Cu") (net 13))
 (segment locked (start 38.82 75.5) (end 38.82 85.43) (width 0.92) (layer "B.Cu") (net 13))
 (segment locked (start 26.12 85.43) (end 28.66 85.43) (width 0.92) (layer "B.Cu") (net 2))
 (segment locked (start 28.66 85.43) (end 28.66 87.25) (width 0.92) (layer "B.Cu") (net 2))
 (segment locked (start 28.66 87.25) (end 29.66 88.25) (width 0.92) (layer "B.Cu") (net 2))
 (segment locked (start 29.66 88.25) (end 40.36 88.25) (width 0.92) (layer "B.Cu") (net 2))
 (segment locked (start 40.36 88.25) (end 41.36 87.25) (width 0.92) (layer "B.Cu") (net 2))
 (segment locked (start 41.36 87.25) (end 41.36 85.43) (width 0.92) (layer "B.Cu") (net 2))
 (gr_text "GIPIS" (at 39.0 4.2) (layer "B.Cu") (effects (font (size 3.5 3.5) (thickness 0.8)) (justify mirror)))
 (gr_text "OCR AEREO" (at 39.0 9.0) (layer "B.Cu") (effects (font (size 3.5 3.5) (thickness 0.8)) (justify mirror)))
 (gr_line (start 0 0) (end 104.0 0) (layer "Edge.Cuts") (width 0.1))
 (gr_line (start 104.0 0) (end 104.0 90.0) (layer "Edge.Cuts") (width 0.1))
 (gr_line (start 104.0 90.0) (end 0 90.0) (layer "Edge.Cuts") (width 0.1))
 (gr_line (start 0 90.0) (end 0 0) (layer "Edge.Cuts") (width 0.1)))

